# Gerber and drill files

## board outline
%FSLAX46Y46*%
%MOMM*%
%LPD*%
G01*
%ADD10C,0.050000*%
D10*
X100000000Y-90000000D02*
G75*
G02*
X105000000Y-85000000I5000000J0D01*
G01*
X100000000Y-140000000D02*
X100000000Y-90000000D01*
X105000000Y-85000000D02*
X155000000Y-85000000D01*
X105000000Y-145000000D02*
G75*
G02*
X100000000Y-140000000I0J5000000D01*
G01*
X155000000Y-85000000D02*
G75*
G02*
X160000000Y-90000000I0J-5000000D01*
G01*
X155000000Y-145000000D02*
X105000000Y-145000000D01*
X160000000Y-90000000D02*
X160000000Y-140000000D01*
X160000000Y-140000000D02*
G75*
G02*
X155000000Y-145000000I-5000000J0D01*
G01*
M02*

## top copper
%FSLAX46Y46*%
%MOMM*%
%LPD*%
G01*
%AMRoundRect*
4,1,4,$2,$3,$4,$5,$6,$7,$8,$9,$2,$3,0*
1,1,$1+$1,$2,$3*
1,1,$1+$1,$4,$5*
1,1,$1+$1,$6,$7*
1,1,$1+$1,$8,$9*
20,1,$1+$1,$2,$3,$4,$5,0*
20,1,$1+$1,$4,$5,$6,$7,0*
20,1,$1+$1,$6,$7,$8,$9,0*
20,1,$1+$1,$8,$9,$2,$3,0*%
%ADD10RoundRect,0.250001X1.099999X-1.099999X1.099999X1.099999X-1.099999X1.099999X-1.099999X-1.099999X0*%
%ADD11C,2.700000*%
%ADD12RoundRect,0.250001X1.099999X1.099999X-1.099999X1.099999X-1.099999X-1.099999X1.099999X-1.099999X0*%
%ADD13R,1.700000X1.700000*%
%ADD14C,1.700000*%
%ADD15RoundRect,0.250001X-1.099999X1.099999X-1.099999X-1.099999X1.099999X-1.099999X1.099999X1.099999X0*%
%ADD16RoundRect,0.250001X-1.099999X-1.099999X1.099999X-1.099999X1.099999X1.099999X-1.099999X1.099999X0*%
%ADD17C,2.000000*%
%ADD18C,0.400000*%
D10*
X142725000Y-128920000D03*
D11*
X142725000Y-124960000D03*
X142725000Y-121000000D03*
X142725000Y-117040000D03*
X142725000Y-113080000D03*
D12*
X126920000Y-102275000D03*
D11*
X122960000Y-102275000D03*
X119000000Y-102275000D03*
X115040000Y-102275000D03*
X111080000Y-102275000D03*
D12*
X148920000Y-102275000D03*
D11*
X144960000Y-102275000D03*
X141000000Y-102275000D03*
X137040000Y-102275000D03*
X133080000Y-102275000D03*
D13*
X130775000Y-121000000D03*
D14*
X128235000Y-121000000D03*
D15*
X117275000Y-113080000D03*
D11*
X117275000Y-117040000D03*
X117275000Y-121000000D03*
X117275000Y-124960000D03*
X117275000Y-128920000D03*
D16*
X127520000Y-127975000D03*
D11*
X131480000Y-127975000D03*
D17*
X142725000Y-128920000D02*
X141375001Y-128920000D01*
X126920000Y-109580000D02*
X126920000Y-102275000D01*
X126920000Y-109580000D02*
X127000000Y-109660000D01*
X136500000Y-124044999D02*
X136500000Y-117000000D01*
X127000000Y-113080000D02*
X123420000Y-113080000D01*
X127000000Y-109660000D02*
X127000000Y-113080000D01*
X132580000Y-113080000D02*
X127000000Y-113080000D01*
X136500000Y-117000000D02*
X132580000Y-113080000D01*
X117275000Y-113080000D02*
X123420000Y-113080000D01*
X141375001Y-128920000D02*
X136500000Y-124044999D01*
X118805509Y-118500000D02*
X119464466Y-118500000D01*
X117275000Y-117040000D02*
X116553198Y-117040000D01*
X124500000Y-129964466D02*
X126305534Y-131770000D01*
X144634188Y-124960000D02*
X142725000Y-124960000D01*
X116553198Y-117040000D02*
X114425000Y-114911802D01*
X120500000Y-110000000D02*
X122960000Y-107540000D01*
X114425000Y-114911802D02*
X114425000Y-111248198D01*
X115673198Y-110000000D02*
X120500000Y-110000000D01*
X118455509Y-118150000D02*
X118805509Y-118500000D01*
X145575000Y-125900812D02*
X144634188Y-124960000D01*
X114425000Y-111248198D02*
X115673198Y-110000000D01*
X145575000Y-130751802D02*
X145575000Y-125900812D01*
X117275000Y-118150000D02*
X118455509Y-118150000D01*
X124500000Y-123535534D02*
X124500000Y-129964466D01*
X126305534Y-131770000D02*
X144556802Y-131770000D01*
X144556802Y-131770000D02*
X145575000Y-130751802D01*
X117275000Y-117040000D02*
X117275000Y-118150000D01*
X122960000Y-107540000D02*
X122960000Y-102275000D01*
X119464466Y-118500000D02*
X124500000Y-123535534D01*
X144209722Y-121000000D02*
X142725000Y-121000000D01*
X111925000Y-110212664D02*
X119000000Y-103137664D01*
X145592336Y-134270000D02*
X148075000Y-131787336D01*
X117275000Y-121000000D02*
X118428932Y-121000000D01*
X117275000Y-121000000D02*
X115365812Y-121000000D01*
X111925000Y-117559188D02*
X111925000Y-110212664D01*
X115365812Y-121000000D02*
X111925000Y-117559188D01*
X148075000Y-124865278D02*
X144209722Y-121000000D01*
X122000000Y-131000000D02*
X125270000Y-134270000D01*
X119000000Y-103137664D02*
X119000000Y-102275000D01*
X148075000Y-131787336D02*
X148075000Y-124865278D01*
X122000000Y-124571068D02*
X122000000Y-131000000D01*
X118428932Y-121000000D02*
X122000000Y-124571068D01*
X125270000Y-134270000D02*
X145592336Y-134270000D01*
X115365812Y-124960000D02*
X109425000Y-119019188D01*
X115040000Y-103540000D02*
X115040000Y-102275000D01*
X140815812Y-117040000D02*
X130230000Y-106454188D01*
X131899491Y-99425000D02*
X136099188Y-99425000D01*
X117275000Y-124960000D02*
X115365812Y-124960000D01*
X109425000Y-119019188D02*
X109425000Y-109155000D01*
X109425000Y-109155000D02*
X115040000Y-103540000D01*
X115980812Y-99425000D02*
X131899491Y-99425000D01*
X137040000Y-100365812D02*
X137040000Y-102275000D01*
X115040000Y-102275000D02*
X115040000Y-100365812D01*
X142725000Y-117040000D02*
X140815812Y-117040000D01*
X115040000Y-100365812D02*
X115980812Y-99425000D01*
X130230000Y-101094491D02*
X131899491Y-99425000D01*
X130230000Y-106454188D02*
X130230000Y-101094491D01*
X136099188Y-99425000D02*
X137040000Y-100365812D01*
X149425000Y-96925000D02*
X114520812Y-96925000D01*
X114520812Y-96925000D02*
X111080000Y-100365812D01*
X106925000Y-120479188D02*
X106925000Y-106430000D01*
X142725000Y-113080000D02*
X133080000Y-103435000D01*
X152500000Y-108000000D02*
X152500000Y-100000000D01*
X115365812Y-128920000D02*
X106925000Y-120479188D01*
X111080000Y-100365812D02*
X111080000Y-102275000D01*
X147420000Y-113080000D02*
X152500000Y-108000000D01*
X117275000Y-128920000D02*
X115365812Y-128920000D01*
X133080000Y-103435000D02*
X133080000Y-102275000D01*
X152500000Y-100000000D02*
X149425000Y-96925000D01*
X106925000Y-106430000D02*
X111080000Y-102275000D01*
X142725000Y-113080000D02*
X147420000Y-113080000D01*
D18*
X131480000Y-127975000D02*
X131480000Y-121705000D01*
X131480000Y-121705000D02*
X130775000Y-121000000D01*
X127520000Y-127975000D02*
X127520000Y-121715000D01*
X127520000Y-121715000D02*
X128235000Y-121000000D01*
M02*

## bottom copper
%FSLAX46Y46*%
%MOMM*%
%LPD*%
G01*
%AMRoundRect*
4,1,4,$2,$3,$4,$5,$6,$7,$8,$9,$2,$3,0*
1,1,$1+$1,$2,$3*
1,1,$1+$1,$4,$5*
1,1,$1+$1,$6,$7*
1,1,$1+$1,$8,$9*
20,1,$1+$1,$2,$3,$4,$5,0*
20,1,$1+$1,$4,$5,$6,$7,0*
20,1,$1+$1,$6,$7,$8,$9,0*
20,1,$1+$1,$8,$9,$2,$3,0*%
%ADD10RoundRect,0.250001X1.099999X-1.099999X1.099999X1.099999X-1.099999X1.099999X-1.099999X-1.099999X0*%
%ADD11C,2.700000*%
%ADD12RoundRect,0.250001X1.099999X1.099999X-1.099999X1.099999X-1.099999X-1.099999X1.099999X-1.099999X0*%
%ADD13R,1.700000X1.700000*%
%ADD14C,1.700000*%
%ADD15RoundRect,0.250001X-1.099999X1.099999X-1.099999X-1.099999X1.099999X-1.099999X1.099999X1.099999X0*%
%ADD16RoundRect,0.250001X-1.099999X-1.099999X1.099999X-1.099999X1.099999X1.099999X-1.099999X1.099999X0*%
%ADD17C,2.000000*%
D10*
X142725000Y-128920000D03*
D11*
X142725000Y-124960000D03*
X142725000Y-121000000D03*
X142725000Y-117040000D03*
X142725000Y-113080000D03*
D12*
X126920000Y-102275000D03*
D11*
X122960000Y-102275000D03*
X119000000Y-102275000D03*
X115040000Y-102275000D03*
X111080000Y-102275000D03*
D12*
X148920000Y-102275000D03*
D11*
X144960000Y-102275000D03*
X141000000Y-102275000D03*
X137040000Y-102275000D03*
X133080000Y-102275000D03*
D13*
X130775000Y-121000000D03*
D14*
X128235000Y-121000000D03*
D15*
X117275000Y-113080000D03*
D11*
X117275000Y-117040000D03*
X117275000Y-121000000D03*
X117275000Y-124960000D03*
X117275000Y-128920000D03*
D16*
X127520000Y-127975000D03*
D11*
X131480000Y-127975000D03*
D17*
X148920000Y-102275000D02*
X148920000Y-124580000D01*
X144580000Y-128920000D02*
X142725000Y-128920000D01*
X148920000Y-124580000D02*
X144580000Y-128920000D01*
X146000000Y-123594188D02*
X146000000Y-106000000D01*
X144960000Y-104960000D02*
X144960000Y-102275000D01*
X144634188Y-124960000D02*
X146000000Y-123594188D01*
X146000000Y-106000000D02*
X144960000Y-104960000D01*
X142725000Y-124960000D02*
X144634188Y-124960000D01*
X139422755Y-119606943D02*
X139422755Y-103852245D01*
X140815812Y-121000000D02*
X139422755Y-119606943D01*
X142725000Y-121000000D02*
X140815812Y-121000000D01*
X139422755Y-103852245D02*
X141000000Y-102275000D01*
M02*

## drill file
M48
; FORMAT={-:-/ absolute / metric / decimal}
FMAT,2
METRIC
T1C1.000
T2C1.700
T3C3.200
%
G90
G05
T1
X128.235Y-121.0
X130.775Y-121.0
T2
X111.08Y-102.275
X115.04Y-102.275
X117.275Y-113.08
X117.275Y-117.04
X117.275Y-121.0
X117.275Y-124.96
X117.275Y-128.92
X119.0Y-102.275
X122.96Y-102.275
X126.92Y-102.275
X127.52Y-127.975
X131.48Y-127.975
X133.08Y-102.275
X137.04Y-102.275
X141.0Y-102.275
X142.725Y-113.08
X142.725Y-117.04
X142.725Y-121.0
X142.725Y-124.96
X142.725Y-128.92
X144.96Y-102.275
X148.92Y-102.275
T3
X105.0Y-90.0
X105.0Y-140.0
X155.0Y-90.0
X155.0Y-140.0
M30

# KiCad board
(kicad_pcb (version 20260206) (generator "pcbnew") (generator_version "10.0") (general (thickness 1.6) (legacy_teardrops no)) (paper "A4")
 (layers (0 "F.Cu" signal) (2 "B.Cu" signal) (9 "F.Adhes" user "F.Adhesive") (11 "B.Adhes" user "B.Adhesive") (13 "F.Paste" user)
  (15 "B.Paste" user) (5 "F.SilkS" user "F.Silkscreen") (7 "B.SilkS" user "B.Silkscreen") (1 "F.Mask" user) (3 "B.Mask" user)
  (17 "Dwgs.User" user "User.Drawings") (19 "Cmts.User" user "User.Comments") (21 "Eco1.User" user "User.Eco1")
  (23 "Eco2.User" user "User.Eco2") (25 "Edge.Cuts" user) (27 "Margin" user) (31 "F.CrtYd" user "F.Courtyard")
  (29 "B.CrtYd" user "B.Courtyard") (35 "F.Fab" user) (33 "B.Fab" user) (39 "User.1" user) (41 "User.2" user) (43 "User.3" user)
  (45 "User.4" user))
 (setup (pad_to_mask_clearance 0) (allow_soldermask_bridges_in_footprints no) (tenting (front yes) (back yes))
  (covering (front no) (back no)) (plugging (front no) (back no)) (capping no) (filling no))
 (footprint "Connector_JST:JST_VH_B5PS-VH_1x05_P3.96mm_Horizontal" (layer "F.Cu") (at 142.725 128.92 90)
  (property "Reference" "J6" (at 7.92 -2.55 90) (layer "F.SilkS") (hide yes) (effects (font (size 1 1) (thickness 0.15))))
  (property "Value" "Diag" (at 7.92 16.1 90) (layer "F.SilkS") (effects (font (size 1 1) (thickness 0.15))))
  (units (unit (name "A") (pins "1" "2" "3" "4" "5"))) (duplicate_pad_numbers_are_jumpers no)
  (pad "1" thru_hole roundrect (at 0 0 90) (size 2.7 2.7) (drill 1.7) (layers "*.Cu" "*.Mask") (remove_unused_layers no)
   (roundrect_rratio 0.092593) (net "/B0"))
  (pad "2" thru_hole circle (at 3.96 0 90) (size 2.7 2.7) (drill 1.7) (layers "*.Cu" "*.Mask") (remove_unused_layers no) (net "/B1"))
  (pad "3" thru_hole circle (at 7.92 0 90) (size 2.7 2.7) (drill 1.7) (layers "*.Cu" "*.Mask") (remove_unused_layers no) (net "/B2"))
  (pad "4" thru_hole circle (at 11.88 0 90) (size 2.7 2.7) (drill 1.7) (layers "*.Cu" "*.Mask") (remove_unused_layers no) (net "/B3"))
  (pad "5" thru_hole circle (at 15.84 0 90) (size 2.7 2.7) (drill 1.7) (layers "*.Cu" "*.Mask") (remove_unused_layers no) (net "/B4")))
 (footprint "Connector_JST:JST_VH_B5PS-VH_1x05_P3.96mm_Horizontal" (layer "F.Cu") (at 126.92 102.275 180)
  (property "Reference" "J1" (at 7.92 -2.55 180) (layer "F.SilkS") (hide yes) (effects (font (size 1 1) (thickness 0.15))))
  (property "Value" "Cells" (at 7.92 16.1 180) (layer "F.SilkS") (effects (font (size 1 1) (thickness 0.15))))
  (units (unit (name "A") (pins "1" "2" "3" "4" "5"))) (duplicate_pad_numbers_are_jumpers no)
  (pad "1" thru_hole roundrect (at 0 0 180) (size 2.7 2.7) (drill 1.7) (layers "*.Cu" "*.Mask") (remove_unused_layers no)
   (roundrect_rratio 0.092593) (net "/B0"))
  (pad "2" thru_hole circle (at 3.96 0 180) (size 2.7 2.7) (drill 1.7) (layers "*.Cu" "*.Mask") (remove_unused_layers no) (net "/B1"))
  (pad "3" thru_hole circle (at 7.92 0 180) (size 2.7 2.7) (drill 1.7) (layers "*.Cu" "*.Mask") (remove_unused_layers no) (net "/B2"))
  (pad "4" thru_hole circle (at 11.88 0 180) (size 2.7 2.7) (drill 1.7) (layers "*.Cu" "*.Mask") (remove_unused_layers no) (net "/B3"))
  (pad "5" thru_hole circle (at 15.84 0 180) (size 2.7 2.7) (drill 1.7) (layers "*.Cu" "*.Mask") (remove_unused_layers no) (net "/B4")))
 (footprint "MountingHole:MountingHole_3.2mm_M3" (layer "F.Cu") (at 105 140)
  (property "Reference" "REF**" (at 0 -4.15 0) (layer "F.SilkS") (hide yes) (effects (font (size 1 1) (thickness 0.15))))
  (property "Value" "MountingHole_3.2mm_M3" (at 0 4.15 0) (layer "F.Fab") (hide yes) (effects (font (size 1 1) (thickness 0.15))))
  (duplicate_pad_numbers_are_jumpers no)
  (pad "" np_thru_hole circle (at 0 0) (size 3.2 3.2) (drill 3.2) (layers "*.Cu" "*.Mask")))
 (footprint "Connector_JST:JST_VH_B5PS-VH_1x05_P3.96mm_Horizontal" (layer "F.Cu") (at 148.92 102.275 180)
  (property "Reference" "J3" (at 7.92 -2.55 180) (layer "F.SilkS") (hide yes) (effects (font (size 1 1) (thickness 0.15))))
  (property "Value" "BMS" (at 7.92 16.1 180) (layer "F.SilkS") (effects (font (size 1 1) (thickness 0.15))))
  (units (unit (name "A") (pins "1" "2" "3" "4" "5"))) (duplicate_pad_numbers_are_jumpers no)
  (pad "1" thru_hole roundrect (at 0 0 180) (size 2.7 2.7) (drill 1.7) (layers "*.Cu" "*.Mask") (remove_unused_layers no)
   (roundrect_rratio 0.092593) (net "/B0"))
  (pad "2" thru_hole circle (at 3.96 0 180) (size 2.7 2.7) (drill 1.7) (layers "*.Cu" "*.Mask") (remove_unused_layers no) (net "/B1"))
  (pad "3" thru_hole circle (at 7.92 0 180) (size 2.7 2.7) (drill 1.7) (layers "*.Cu" "*.Mask") (remove_unused_layers no) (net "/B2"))
  (pad "4" thru_hole circle (at 11.88 0 180) (size 2.7 2.7) (drill 1.7) (layers "*.Cu" "*.Mask") (remove_unused_layers no) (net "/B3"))
  (pad "5" thru_hole circle (at 15.84 0 180) (size 2.7 2.7) (drill 1.7) (layers "*.Cu" "*.Mask") (remove_unused_layers no) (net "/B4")))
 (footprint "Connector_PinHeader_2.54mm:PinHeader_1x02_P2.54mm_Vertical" (layer "F.Cu") (at 130.775 121 -90)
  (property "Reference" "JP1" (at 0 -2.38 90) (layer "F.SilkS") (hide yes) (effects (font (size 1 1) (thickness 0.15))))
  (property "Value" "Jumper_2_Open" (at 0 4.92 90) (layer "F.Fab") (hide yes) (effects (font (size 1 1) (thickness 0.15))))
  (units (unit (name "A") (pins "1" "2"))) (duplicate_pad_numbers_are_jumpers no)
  (pad "1" thru_hole rect (at 0 0 270) (size 1.7 1.7) (drill 1) (layers "*.Cu" "*.Mask") (remove_unused_layers no) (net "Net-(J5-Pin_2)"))
  (pad "2" thru_hole circle (at 0 2.54 270) (size 1.7 1.7) (drill 1) (layers "*.Cu" "*.Mask") (remove_unused_layers no)
   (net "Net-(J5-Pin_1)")))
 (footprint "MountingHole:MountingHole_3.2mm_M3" (layer "F.Cu") (at 105 90)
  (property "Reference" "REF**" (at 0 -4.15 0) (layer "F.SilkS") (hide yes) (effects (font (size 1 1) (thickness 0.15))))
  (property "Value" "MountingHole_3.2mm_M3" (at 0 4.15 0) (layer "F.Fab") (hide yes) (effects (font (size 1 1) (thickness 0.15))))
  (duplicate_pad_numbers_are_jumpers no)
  (pad "" np_thru_hole circle (at 0 0) (size 3.2 3.2) (drill 3.2) (layers "*.Cu" "*.Mask")))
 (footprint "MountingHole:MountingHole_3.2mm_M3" (layer "F.Cu") (at 155 90)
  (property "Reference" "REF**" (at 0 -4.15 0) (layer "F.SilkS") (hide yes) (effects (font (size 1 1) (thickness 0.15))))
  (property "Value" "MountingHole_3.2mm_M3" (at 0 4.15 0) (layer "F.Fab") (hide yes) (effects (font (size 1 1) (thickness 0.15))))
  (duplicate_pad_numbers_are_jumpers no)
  (pad "" np_thru_hole circle (at 0 0) (size 3.2 3.2) (drill 3.2) (layers "*.Cu" "*.Mask")))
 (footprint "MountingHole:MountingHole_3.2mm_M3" (layer "F.Cu") (at 155 140)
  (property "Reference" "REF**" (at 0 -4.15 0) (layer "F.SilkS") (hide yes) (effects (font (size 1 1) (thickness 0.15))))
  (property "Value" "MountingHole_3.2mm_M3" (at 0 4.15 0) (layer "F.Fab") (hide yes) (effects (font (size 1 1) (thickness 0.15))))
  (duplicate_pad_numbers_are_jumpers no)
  (pad "" np_thru_hole circle (at 0 0) (size 3.2 3.2) (drill 3.2) (layers "*.Cu" "*.Mask")))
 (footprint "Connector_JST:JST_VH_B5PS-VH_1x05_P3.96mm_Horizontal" (layer "F.Cu") (at 117.275 113.08 -90)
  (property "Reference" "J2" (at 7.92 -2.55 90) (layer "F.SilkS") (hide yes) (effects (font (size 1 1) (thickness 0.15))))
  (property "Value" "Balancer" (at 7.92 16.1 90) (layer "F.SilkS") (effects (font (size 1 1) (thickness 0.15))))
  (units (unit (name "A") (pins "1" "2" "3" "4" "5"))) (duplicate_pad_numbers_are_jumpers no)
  (pad "1" thru_hole roundrect (at 0 0 270) (size 2.7 2.7) (drill 1.7) (layers "*.Cu" "*.Mask") (remove_unused_layers no)
   (roundrect_rratio 0.092593) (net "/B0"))
  (pad "2" thru_hole circle (at 3.96 0 270) (size 2.7 2.7) (drill 1.7) (layers "*.Cu" "*.Mask") (remove_unused_layers no) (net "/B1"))
  (pad "3" thru_hole circle (at 7.92 0 270) (size 2.7 2.7) (drill 1.7) (layers "*.Cu" "*.Mask") (remove_unused_layers no) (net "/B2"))
  (pad "4" thru_hole circle (at 11.88 0 270) (size 2.7 2.7) (drill 1.7) (layers "*.Cu" "*.Mask") (remove_unused_layers no) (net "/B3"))
  (pad "5" thru_hole circle (at 15.84 0 270) (size 2.7 2.7) (drill 1.7) (layers "*.Cu" "*.Mask") (remove_unused_layers no) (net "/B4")))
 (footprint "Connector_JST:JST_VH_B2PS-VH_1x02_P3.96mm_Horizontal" (layer "F.Cu") (at 127.52 127.975)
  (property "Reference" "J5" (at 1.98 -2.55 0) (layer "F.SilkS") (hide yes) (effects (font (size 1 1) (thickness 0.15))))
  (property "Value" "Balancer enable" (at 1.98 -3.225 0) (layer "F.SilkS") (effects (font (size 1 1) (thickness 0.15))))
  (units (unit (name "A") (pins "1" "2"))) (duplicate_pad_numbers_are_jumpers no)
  (pad "1" thru_hole roundrect (at 0 0) (size 2.7 2.7) (drill 1.7) (layers "*.Cu" "*.Mask") (remove_unused_layers no)
   (roundrect_rratio 0.092593) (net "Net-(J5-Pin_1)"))
  (pad "2" thru_hole circle (at 3.96 0) (size 2.7 2.7) (drill 1.7) (layers "*.Cu" "*.Mask") (remove_unused_layers no) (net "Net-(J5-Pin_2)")))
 (gr_arc (start 100 90) (mid 101.464466 86.464466) (end 105 85) (stroke (width 0.05) (type default)) (layer "Edge.Cuts"))
 (gr_line (start 100 140) (end 100 90) (stroke (width 0.05) (type default)) (layer "Edge.Cuts"))
 (gr_line (start 105 85) (end 155 85) (stroke (width 0.05) (type default)) (layer "Edge.Cuts"))
 (gr_arc (start 105 145) (mid 101.464466 143.535534) (end 100 140) (stroke (width 0.05) (type solid)) (layer "Edge.Cuts"))
 (gr_arc (start 155 85) (mid 158.535534 86.464466) (end 160 90) (stroke (width 0.05) (type default)) (layer "Edge.Cuts"))
 (gr_line (start 155 145) (end 105 145) (stroke (width 0.05) (type solid)) (layer "Edge.Cuts"))
 (gr_line (start 160 90) (end 160 140) (stroke (width 0.05) (type solid)) (layer "Edge.Cuts"))
 (gr_arc (start 160 140) (mid 158.535534 143.535534) (end 155 145) (stroke (width 0.05) (type solid)) (layer "Edge.Cuts"))
 (segment (start 142.725 128.92) (end 141.375001 128.92) (width 2) (layer "F.Cu") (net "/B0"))
 (segment (start 126.92 109.58) (end 126.92 102.275) (width 2) (layer "F.Cu") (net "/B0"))
 (segment (start 126.92 109.58) (end 127 109.66) (width 2) (layer "F.Cu") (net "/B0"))
 (segment (start 136.5 124.044999) (end 136.5 117) (width 2) (layer "F.Cu") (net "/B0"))
 (segment (start 127 113.08) (end 123.42 113.08) (width 2) (layer "F.Cu") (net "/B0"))
 (segment (start 127 109.66) (end 127 113.08) (width 2) (layer "F.Cu") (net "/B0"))
 (segment (start 132.58 113.08) (end 127 113.08) (width 2) (layer "F.Cu") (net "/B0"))
 (segment (start 136.5 117) (end 132.58 113.08) (width 2) (layer "F.Cu") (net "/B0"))
 (segment (start 117.275 113.08) (end 123.42 113.08) (width 2) (layer "F.Cu") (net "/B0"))
 (segment (start 141.375001 128.92) (end 136.5 124.044999) (width 2) (layer "F.Cu") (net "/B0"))
 (segment (start 148.92 102.275) (end 148.92 124.58) (width 2) (layer "B.Cu") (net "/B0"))
 (segment (start 144.58 128.92) (end 142.725 128.92) (width 2) (layer "B.Cu") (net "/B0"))
 (segment (start 148.92 124.58) (end 144.58 128.92) (width 2) (layer "B.Cu") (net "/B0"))
 (segment (start 118.805509 118.5) (end 119.464466 118.5) (width 2) (layer "F.Cu") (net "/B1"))
 (segment (start 117.275 117.04) (end 116.553198 117.04) (width 2) (layer "F.Cu") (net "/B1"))
 (segment (start 124.5 129.964466) (end 126.305534 131.77) (width 2) (layer "F.Cu") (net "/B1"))
 (segment (start 144.634188 124.96) (end 142.725 124.96) (width 2) (layer "F.Cu") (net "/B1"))
 (segment (start 116.553198 117.04) (end 114.425 114.911802) (width 2) (layer "F.Cu") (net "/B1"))
 (segment (start 120.5 110) (end 122.96 107.54) (width 2) (layer "F.Cu") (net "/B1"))
 (segment (start 114.425 114.911802) (end 114.425 111.248198) (width 2) (layer "F.Cu") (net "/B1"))
 (segment (start 115.673198 110) (end 120.5 110) (width 2) (layer "F.Cu") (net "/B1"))
 (segment (start 118.455509 118.15) (end 118.805509 118.5) (width 2) (layer "F.Cu") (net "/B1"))
 (segment (start 145.575 125.900812) (end 144.634188 124.96) (width 2) (layer "F.Cu") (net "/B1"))
 (segment (start 114.425 111.248198) (end 115.673198 110) (width 2) (layer "F.Cu") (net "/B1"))
 (segment (start 145.575 130.751802) (end 145.575 125.900812) (width 2) (layer "F.Cu") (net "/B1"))
 (segment (start 117.275 118.15) (end 118.455509 118.15) (width 2) (layer "F.Cu") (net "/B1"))
 (segment (start 124.5 123.535534) (end 124.5 129.964466) (width 2) (layer "F.Cu") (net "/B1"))
 (segment (start 126.305534 131.77) (end 144.556802 131.77) (width 2) (layer "F.Cu") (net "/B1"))
 (segment (start 144.556802 131.77) (end 145.575 130.751802) (width 2) (layer "F.Cu") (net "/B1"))
 (segment (start 117.275 117.04) (end 117.275 118.15) (width 2) (layer "F.Cu") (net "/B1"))
 (segment (start 122.96 107.54) (end 122.96 102.275) (width 2) (layer "F.Cu") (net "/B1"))
 (segment (start 119.464466 118.5) (end 124.5 123.535534) (width 2) (layer "F.Cu") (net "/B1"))
 (segment (start 146 123.594188) (end 146 106) (width 2) (layer "B.Cu") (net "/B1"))
 (segment (start 144.96 104.96) (end 144.96 102.275) (width 2) (layer "B.Cu") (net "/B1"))
 (segment (start 144.634188 124.96) (end 146 123.594188) (width 2) (layer "B.Cu") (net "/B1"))
 (segment (start 146 106) (end 144.96 104.96) (width 2) (layer "B.Cu") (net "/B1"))
 (segment (start 142.725 124.96) (end 144.634188 124.96) (width 2) (layer "B.Cu") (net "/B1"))
 (segment (start 144.209722 121) (end 142.725 121) (width 2) (layer "F.Cu") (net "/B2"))
 (segment (start 111.925 110.212664) (end 119 103.137664) (width 2) (layer "F.Cu") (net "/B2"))
 (segment (start 145.592336 134.27) (end 148.075 131.787336) (width 2) (layer "F.Cu") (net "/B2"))
 (segment (start 117.275 121) (end 118.428932 121) (width 2) (layer "F.Cu") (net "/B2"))
 (segment (start 117.275 121) (end 115.365812 121) (width 2) (layer "F.Cu") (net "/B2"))
 (segment (start 111.925 117.559188) (end 111.925 110.212664) (width 2) (layer "F.Cu") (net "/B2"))
 (segment (start 115.365812 121) (end 111.925 117.559188) (width 2) (layer "F.Cu") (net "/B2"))
 (segment (start 148.075 124.865278) (end 144.209722 121) (width 2) (layer "F.Cu") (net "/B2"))
 (segment (start 122 131) (end 125.27 134.27) (width 2) (layer "F.Cu") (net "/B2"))
 (segment (start 119 103.137664) (end 119 102.275) (width 2) (layer "F.Cu") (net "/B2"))
 (segment (start 148.075 131.787336) (end 148.075 124.865278) (width 2) (layer "F.Cu") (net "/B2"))
 (segment (start 122 124.571068) (end 122 131) (width 2) (layer "F.Cu") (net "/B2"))
 (segment (start 118.428932 121) (end 122 124.571068) (width 2) (layer "F.Cu") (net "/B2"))
 (segment (start 125.27 134.27) (end 145.592336 134.27) (width 2) (layer "F.Cu") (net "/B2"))
 (segment (start 139.422755 119.606943) (end 139.422755 103.852245) (width 2) (layer "B.Cu") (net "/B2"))
 (segment (start 140.815812 121) (end 139.422755 119.606943) (width 2) (layer "B.Cu") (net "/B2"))
 (segment (start 142.725 121) (end 140.815812 121) (width 2) (layer "B.Cu") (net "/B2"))
 (segment (start 139.422755 103.852245) (end 141 102.275) (width 2) (layer "B.Cu") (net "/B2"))
 (segment (start 115.365812 124.96) (end 109.425 119.019188) (width 2) (layer "F.Cu") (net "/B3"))
 (segment (start 115.04 103.54) (end 115.04 102.275) (width 2) (layer "F.Cu") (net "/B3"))
 (segment (start 140.815812 117.04) (end 130.23 106.454188) (width 2) (layer "F.Cu") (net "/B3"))
 (segment (start 131.899491 99.425) (end 136.099188 99.425) (width 2) (layer "F.Cu") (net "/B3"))
 (segment (start 117.275 124.96) (end 115.365812 124.96) (width 2) (layer "F.Cu") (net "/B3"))
 (segment (start 109.425 119.019188) (end 109.425 109.155) (width 2) (layer "F.Cu") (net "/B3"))
 (segment (start 109.425 109.155) (end 115.04 103.54) (width 2) (layer "F.Cu") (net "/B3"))
 (segment (start 115.980812 99.425) (end 131.899491 99.425) (width 2) (layer "F.Cu") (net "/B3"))
 (segment (start 137.04 100.365812) (end 137.04 102.275) (width 2) (layer "F.Cu") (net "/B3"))
 (segment (start 115.04 102.275) (end 115.04 100.365812) (width 2) (layer "F.Cu") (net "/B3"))
 (segment (start 142.725 117.04) (end 140.815812 117.04) (width 2) (layer "F.Cu") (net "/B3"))
 (segment (start 115.04 100.365812) (end 115.980812 99.425) (width 2) (layer "F.Cu") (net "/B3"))
 (segment (start 130.23 101.094491) (end 131.899491 99.425) (width 2) (layer "F.Cu") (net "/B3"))
 (segment (start 130.23 106.454188) (end 130.23 101.094491) (width 2) (layer "F.Cu") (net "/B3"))
 (segment (start 136.099188 99.425) (end 137.04 100.365812) (width 2) (layer "F.Cu") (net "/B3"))
 (segment (start 149.425 96.925) (end 114.520812 96.925) (width 2) (layer "F.Cu") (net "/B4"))
 (segment (start 114.520812 96.925) (end 111.08 100.365812) (width 2) (layer "F.Cu") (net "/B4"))
 (segment (start 106.925 120.479188) (end 106.925 106.43) (width 2) (layer "F.Cu") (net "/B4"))
 (segment (start 142.725 113.08) (end 133.08 103.435) (width 2) (layer "F.Cu") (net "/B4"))
 (segment (start 152.5 108) (end 152.5 100) (width 2) (layer "F.Cu") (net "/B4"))
 (segment (start 115.365812 128.92) (end 106.925 120.479188) (width 2) (layer "F.Cu") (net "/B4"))
 (segment (start 111.08 100.365812) (end 111.08 102.275) (width 2) (layer "F.Cu") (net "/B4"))
 (segment (start 147.42 113.08) (end 152.5 108) (width 2) (layer "F.Cu") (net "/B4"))
 (segment (start 117.275 128.92) (end 115.365812 128.92) (width 2) (layer "F.Cu") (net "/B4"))
 (segment (start 133.08 103.435) (end 133.08 102.275) (width 2) (layer "F.Cu") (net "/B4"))
 (segment (start 152.5 100) (end 149.425 96.925) (width 2) (layer "F.Cu") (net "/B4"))
 (segment (start 106.925 106.43) (end 111.08 102.275) (width 2) (layer "F.Cu") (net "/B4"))
 (segment (start 142.725 113.08) (end 147.42 113.08) (width 2) (layer "F.Cu") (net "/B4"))
 (segment (start 131.48 127.975) (end 131.48 121.705) (width 0.4) (layer "F.Cu") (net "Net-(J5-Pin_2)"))
 (segment (start 131.48 121.705) (end 130.775 121) (width 0.4) (layer "F.Cu") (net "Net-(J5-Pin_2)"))
 (segment (start 127.52 127.975) (end 127.52 121.715) (width 0.4) (layer "F.Cu") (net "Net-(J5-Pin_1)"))
 (segment (start 127.52 121.715) (end 128.235 121) (width 0.4) (layer "F.Cu") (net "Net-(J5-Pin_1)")))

